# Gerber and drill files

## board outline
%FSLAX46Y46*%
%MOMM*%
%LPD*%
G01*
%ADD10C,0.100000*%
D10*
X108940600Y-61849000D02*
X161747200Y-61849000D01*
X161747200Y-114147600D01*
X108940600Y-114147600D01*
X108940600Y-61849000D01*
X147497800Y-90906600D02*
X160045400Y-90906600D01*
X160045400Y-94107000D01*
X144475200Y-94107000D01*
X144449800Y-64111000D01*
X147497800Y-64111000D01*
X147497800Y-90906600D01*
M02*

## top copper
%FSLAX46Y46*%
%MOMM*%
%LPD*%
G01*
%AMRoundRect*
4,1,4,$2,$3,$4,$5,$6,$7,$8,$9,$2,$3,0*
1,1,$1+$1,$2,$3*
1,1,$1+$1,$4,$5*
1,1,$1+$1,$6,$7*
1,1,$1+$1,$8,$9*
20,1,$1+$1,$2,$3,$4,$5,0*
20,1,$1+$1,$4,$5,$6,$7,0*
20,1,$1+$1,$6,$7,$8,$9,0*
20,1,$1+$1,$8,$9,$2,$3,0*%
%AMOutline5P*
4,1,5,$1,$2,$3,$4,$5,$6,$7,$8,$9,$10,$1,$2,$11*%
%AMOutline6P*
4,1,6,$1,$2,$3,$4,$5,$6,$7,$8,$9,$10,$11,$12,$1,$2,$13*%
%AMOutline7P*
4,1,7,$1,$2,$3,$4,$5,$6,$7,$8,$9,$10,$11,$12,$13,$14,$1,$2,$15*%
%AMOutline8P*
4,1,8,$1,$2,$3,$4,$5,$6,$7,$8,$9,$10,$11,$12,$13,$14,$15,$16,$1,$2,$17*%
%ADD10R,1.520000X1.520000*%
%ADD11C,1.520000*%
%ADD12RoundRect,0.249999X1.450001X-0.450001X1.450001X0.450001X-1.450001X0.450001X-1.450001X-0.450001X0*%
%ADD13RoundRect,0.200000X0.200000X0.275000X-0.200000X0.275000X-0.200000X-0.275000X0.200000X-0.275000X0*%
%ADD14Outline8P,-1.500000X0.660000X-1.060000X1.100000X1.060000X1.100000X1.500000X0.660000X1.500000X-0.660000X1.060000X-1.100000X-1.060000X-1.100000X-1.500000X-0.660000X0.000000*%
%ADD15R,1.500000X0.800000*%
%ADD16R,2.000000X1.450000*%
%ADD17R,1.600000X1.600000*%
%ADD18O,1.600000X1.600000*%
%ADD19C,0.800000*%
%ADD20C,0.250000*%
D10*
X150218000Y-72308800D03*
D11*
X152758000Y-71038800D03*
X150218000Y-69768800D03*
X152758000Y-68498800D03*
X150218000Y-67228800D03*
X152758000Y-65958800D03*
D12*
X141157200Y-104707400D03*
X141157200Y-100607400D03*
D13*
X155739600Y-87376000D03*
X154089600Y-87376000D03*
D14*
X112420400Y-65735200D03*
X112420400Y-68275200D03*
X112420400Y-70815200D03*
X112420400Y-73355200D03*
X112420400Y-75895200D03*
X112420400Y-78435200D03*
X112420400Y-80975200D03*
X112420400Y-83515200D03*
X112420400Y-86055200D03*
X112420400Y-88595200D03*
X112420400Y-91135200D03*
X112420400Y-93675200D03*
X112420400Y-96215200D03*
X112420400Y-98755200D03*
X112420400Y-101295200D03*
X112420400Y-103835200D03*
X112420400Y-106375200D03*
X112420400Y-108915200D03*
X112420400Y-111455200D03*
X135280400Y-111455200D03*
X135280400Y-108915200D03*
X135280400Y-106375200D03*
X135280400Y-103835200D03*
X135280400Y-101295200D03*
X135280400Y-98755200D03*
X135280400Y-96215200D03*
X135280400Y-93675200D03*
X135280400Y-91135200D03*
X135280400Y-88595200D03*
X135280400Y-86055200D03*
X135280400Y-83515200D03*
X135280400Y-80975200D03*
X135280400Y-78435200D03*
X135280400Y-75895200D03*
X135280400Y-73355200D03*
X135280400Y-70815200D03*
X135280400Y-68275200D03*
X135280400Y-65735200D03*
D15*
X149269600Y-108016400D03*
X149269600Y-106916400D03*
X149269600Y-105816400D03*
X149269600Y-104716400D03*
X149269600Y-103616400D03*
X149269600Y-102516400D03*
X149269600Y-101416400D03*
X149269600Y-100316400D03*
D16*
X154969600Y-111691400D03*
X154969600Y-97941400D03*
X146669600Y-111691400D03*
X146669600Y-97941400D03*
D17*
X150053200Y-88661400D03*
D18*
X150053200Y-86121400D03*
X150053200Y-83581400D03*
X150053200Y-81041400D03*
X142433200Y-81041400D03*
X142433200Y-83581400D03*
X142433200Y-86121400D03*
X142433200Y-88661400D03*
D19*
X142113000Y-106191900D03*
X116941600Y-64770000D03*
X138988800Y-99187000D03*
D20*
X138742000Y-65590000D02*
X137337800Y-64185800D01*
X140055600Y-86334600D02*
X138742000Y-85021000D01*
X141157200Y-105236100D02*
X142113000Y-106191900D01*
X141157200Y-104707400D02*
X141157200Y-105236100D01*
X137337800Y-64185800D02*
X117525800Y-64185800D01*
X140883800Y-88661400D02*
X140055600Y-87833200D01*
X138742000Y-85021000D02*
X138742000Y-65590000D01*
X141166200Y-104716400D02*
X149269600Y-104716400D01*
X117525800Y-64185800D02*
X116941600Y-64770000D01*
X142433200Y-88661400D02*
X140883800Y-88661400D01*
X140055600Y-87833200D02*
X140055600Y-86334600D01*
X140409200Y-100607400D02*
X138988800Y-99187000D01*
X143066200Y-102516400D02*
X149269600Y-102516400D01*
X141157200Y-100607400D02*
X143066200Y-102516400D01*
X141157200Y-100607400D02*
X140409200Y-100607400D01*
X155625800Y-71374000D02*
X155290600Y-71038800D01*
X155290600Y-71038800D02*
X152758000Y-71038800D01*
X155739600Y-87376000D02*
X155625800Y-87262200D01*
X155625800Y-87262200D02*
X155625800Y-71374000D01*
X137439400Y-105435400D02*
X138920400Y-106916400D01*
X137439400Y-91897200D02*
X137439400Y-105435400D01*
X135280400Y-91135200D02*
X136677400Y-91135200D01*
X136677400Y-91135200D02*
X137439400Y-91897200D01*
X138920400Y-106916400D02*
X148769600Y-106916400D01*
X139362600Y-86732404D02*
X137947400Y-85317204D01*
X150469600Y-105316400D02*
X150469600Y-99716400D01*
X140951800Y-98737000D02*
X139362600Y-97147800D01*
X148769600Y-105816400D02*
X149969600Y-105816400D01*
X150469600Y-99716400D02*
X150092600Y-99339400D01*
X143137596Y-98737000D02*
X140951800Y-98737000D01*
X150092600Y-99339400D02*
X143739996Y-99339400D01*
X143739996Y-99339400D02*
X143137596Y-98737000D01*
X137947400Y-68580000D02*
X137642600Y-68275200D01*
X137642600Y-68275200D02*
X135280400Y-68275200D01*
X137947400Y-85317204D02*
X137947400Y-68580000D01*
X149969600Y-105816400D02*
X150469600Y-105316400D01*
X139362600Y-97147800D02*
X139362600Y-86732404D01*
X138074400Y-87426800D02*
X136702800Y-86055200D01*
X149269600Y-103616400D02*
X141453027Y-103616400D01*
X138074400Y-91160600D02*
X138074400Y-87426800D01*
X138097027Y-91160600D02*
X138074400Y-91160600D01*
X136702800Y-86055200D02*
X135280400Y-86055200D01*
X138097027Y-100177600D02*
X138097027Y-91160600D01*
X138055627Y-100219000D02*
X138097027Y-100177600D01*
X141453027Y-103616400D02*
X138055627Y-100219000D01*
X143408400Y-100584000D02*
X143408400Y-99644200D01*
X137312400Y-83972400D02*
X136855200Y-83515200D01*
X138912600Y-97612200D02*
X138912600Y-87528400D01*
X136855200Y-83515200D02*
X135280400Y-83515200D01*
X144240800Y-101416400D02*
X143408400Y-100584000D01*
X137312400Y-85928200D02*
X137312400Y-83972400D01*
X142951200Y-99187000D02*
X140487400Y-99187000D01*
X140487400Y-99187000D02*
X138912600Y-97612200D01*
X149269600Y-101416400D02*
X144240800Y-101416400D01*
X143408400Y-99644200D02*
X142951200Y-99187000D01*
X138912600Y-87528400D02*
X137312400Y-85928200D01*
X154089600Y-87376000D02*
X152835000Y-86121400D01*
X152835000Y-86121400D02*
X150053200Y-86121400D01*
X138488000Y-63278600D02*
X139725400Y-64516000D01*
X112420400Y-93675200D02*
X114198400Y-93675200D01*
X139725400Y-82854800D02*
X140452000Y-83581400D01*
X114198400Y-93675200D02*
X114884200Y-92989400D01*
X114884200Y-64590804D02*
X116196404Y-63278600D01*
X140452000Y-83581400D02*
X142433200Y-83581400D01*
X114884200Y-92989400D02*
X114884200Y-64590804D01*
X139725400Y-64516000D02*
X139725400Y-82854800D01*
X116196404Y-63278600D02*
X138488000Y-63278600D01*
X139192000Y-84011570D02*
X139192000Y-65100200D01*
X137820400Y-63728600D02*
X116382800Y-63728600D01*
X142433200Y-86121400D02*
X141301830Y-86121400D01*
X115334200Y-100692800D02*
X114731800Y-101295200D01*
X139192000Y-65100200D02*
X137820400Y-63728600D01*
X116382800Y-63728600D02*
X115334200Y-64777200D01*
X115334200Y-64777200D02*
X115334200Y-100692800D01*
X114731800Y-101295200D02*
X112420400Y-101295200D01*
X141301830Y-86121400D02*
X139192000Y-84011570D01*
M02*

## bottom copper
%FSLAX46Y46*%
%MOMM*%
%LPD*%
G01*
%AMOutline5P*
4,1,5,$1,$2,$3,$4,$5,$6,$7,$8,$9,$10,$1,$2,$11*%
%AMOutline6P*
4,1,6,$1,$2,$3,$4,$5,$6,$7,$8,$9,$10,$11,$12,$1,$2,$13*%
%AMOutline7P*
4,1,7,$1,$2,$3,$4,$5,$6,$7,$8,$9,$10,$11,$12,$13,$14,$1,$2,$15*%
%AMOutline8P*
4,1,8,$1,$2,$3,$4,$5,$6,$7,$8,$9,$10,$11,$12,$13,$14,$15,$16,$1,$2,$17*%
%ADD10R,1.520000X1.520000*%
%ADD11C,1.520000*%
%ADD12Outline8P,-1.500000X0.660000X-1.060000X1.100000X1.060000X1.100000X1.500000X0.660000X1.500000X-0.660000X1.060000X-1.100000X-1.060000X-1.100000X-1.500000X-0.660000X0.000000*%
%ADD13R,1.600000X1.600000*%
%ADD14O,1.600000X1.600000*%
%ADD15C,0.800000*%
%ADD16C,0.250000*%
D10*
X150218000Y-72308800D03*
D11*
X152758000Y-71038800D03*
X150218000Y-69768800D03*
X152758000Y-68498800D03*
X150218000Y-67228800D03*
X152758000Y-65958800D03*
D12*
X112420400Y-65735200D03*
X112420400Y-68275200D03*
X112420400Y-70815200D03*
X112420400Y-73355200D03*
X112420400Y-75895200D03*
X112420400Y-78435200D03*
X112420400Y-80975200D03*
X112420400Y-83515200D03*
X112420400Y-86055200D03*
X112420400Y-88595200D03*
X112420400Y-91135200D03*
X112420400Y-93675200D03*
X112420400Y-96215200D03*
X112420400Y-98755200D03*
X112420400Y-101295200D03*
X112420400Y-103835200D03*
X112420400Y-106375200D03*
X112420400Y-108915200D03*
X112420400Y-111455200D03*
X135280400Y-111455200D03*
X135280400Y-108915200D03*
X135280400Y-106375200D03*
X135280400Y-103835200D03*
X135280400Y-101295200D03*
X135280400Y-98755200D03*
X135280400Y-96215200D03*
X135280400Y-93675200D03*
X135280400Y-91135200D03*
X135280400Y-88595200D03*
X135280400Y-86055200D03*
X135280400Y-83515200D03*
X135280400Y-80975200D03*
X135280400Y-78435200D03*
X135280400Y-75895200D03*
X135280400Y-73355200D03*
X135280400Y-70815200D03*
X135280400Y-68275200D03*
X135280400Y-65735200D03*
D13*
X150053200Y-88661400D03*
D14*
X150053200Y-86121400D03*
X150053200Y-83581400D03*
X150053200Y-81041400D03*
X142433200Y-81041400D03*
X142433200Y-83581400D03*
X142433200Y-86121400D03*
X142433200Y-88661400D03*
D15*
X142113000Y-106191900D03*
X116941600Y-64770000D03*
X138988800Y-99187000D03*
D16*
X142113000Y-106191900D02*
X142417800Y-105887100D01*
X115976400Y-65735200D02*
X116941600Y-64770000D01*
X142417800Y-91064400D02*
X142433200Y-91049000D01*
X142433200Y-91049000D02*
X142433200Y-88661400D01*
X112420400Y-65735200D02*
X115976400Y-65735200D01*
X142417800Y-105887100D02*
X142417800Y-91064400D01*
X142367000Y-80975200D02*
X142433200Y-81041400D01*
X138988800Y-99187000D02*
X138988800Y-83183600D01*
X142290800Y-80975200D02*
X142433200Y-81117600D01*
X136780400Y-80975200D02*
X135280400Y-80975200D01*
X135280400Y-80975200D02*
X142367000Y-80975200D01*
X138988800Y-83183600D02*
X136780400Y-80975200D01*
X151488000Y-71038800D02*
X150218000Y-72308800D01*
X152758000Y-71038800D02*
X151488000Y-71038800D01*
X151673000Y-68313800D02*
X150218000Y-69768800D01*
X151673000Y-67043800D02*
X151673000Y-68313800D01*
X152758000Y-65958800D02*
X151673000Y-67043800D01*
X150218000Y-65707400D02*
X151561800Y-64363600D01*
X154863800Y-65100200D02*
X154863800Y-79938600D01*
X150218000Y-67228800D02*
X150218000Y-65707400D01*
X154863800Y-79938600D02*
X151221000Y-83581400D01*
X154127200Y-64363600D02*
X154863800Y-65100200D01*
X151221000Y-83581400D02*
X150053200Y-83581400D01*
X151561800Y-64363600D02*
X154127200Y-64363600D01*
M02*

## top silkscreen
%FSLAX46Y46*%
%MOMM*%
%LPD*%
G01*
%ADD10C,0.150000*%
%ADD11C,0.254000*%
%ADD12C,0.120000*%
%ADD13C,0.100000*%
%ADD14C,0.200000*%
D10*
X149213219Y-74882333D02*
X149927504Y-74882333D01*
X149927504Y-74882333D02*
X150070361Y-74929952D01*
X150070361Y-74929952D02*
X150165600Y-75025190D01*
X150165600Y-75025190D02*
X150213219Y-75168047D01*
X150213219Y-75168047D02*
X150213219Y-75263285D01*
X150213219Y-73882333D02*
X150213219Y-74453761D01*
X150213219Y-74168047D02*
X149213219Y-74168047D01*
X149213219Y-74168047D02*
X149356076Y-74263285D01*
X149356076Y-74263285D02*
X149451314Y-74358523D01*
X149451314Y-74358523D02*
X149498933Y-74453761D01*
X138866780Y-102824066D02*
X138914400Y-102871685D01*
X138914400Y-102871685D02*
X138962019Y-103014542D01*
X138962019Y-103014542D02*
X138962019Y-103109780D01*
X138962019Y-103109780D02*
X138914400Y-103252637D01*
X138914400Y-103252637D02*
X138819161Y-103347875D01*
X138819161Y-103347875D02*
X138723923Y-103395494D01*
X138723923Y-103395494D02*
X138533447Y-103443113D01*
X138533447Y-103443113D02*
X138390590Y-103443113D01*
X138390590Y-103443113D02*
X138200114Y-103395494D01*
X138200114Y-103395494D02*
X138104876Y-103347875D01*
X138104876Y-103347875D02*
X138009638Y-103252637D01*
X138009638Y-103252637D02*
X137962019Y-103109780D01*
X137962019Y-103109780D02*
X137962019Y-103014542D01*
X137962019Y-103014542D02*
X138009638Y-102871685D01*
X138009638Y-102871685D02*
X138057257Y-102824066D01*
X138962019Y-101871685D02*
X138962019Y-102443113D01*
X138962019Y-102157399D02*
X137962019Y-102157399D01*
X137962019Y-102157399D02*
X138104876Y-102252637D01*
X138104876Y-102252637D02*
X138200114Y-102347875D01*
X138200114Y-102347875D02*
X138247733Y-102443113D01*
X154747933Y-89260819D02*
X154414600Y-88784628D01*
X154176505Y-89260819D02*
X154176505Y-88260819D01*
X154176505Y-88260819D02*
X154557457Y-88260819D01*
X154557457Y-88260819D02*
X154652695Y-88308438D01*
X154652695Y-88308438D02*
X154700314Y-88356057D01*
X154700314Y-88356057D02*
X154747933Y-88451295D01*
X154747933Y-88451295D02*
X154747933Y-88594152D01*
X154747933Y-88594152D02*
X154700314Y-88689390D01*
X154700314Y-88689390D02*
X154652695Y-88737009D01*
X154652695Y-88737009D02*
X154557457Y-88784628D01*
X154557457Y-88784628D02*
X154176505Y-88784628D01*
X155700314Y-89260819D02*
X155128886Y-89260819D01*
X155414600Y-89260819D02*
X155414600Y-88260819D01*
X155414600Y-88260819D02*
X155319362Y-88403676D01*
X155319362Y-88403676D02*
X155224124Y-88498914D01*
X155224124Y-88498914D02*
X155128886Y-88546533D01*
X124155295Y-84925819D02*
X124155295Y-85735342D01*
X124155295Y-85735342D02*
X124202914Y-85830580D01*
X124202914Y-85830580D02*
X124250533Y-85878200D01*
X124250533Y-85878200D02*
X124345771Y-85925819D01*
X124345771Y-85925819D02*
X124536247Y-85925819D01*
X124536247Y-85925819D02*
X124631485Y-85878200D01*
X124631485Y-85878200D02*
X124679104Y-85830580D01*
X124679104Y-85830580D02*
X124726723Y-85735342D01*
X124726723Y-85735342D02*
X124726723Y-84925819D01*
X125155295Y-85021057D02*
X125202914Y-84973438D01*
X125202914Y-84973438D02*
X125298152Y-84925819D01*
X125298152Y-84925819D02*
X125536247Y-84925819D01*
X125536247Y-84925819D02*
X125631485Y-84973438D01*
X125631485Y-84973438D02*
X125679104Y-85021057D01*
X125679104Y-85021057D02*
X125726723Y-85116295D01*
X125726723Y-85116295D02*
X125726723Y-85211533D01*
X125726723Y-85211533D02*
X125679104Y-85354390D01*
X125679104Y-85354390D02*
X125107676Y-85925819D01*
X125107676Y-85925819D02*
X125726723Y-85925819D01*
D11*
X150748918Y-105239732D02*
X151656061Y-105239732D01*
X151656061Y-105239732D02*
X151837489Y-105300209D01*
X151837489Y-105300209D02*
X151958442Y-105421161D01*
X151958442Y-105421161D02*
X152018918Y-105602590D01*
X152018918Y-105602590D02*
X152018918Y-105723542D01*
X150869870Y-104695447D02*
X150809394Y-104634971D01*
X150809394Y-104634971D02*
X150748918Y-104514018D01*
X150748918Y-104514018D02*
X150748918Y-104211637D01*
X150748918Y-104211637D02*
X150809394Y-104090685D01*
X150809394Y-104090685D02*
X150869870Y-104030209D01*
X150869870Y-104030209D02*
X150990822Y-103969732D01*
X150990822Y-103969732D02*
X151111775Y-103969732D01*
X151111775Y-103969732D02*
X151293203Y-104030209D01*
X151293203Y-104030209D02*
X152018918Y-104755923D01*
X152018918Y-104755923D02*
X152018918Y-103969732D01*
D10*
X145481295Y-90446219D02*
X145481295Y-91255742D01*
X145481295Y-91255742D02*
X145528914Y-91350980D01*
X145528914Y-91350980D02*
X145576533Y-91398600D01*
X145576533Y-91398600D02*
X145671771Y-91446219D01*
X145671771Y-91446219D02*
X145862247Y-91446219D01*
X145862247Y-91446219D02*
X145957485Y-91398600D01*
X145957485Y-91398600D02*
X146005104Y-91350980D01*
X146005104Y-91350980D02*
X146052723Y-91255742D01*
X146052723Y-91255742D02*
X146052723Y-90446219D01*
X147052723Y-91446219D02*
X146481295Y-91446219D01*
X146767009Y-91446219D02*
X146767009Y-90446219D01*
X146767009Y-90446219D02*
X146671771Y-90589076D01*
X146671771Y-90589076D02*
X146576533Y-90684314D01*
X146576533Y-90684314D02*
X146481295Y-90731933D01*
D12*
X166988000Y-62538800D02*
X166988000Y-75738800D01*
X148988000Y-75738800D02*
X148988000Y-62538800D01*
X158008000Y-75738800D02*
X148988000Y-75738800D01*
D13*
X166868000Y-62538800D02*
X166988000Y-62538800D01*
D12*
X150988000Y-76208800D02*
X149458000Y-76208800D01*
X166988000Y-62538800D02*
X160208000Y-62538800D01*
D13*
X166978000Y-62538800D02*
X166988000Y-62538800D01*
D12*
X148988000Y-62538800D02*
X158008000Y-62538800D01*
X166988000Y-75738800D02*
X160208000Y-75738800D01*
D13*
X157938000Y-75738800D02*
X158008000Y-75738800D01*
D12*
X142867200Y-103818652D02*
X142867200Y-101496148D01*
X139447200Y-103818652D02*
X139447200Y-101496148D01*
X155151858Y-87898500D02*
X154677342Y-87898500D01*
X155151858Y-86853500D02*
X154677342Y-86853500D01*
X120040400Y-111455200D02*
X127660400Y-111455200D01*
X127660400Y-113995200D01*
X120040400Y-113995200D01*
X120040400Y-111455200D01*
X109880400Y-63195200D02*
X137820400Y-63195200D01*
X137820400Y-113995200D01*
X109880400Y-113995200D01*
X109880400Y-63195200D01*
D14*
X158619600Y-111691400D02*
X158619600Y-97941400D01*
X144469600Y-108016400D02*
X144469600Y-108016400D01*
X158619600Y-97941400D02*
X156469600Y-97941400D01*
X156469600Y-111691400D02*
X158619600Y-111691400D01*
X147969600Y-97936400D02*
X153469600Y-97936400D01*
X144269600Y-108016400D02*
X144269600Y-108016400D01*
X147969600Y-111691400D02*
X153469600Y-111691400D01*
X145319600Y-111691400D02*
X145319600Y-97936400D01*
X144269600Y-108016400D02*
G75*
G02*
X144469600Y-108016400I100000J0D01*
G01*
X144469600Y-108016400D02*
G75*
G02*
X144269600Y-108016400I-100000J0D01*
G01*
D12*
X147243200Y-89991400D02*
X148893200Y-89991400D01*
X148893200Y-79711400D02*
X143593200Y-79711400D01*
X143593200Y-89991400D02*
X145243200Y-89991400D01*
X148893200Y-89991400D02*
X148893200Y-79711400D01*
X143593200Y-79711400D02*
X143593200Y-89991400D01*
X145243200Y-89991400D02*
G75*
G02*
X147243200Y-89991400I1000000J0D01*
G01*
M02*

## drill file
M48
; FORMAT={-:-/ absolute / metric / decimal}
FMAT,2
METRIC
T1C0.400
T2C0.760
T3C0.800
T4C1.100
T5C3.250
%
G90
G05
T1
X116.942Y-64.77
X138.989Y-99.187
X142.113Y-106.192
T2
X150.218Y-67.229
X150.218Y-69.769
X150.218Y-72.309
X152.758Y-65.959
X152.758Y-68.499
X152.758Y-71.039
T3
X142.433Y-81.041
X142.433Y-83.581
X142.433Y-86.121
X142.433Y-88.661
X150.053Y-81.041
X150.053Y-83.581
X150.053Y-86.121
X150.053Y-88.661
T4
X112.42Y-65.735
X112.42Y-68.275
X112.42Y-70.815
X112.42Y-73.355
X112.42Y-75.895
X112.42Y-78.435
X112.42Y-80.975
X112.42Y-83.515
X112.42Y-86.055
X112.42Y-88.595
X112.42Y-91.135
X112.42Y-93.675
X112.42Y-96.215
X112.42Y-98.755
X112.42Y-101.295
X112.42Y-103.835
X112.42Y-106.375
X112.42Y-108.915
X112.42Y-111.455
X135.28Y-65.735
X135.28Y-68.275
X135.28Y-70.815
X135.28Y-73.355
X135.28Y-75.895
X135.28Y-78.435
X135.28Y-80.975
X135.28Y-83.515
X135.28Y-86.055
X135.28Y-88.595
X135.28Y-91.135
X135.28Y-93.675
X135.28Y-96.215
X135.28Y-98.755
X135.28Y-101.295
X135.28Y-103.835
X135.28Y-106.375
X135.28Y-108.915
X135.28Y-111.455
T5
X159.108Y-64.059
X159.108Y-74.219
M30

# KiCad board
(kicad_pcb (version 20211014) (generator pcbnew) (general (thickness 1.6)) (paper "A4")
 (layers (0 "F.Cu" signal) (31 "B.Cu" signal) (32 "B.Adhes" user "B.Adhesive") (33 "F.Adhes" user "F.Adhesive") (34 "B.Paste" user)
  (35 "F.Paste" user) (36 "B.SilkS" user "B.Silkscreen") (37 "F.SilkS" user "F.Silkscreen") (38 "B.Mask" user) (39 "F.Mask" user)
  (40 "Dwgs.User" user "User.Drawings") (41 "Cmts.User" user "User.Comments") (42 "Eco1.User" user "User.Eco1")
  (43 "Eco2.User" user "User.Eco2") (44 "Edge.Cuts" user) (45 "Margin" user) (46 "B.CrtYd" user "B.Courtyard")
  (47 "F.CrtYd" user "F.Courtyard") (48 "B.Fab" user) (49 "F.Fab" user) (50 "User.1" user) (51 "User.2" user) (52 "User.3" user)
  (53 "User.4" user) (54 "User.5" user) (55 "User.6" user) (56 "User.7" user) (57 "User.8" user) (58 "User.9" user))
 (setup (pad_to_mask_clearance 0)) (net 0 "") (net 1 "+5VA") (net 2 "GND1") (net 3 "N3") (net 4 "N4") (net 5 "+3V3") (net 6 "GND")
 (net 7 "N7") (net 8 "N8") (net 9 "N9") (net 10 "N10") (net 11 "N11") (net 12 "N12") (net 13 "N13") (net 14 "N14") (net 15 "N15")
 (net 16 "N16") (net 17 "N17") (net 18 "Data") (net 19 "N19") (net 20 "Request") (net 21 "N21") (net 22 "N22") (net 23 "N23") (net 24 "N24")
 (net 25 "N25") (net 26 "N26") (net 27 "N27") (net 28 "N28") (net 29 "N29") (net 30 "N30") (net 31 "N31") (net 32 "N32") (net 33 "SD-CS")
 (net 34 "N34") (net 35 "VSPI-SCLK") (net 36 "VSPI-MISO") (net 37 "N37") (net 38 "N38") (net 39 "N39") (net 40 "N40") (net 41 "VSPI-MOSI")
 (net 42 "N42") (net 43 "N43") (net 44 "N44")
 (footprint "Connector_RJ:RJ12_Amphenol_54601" (layer "F.Cu") (at 150.218 72.3088 90)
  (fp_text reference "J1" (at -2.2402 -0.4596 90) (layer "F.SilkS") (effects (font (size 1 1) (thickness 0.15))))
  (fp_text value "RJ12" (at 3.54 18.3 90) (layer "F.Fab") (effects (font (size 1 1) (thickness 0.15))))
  (fp_line (start 9.77 16.77) (end -3.43 16.77) (layer "F.SilkS") (width 0.12))
  (fp_line (start -3.43 -1.23) (end 9.77 -1.23) (layer "F.SilkS") (width 0.12))
  (fp_line (start -3.43 7.79) (end -3.43 -1.23) (layer "F.SilkS") (width 0.12))
  (fp_line (start 9.77 16.65) (end 9.77 16.77) (layer "F.SilkS") (width 0.1))
  (fp_line (start -3.9 0.77) (end -3.9 -0.76) (layer "F.SilkS") (width 0.12))
  (fp_line (start 9.77 16.77) (end 9.77 9.99) (layer "F.SilkS") (width 0.12))
  (fp_line (start 9.77 16.76) (end 9.77 16.77) (layer "F.SilkS") (width 0.1))
  (fp_line (start 9.77 -1.23) (end 9.77 7.79) (layer "F.SilkS") (width 0.12))
  (fp_line (start -3.43 16.77) (end -3.43 9.99) (layer "F.SilkS") (width 0.12))
  (fp_line (start -3.43 7.72) (end -3.43 7.79) (layer "F.SilkS") (width 0.1))
  (pad "" np_thru_hole circle (at -1.91 8.89 90) (size 3.25 3.25) (drill 3.25) (layers *.Cu *.Mask))
  (pad "" np_thru_hole circle (at 8.25 8.89 90) (size 3.25 3.25) (drill 3.25) (layers *.Cu *.Mask))
  (pad "1" thru_hole rect (at 0 0 90) (size 1.52 1.52) (drill 0.76) (layers *.Cu *.Mask) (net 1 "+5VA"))
  (pad "2" thru_hole circle (at 1.27 2.54 90) (size 1.52 1.52) (drill 0.76) (layers *.Cu *.Mask) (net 1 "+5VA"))
  (pad "3" thru_hole circle (at 2.54 0 90) (size 1.52 1.52) (drill 0.76) (layers *.Cu *.Mask) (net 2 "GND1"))
  (pad "4" thru_hole circle (at 3.81 2.54 90) (size 1.52 1.52) (drill 0.76) (layers *.Cu *.Mask) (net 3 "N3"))
  (pad "5" thru_hole circle (at 5.08 0 90) (size 1.52 1.52) (drill 0.76) (layers *.Cu *.Mask) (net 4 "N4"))
  (pad "6" thru_hole circle (at 6.35 2.54 90) (size 1.52 1.52) (drill 0.76) (layers *.Cu *.Mask) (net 2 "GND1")))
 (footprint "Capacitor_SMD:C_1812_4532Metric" (layer "F.Cu") (at 141.1572 102.6574 90)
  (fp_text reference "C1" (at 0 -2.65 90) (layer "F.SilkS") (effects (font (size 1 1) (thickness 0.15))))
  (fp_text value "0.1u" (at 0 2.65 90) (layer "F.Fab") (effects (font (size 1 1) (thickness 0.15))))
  (fp_line (start -1.161252 1.71) (end 1.161252 1.71) (layer "F.SilkS") (width 0.12))
  (fp_line (start -1.161252 -1.71) (end 1.161252 -1.71) (layer "F.SilkS") (width 0.12))
  (pad "1" smd roundrect (at -2.05 0 90) (size 1.4 3.4) (layers "F.Cu" "F.Paste" "F.Mask") (roundrect_rratio 0.178571) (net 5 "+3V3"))
  (pad "2" smd roundrect (at 2.05 0 90) (size 1.4 3.4) (layers "F.Cu" "F.Paste" "F.Mask") (roundrect_rratio 0.178571) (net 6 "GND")))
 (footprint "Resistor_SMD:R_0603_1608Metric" (layer "F.Cu") (at 154.9146 87.376 180)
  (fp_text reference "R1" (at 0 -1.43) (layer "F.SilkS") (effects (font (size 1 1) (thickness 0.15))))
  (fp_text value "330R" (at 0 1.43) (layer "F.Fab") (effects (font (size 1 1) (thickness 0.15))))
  (fp_line (start -0.237258 -0.5225) (end 0.237258 -0.5225) (layer "F.SilkS") (width 0.12))
  (fp_line (start -0.237258 0.5225) (end 0.237258 0.5225) (layer "F.SilkS") (width 0.12))
  (pad "1" smd roundrect (at -0.825 0 180) (size 0.8 0.95) (layers "F.Cu" "F.Paste" "F.Mask") (roundrect_rratio 0.25) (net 1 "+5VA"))
  (pad "2" smd roundrect (at 0.825 0 180) (size 0.8 0.95) (layers "F.Cu" "F.Paste" "F.Mask") (roundrect_rratio 0.25) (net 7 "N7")))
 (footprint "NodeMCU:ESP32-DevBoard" (layer "F.Cu") (at 112.4204 80.9752)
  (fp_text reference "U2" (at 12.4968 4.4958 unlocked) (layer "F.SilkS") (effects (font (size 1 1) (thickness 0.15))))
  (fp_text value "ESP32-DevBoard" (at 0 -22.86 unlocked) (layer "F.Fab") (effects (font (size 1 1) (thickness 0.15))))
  (fp_rect (start 7.62 30.48) (end 15.24 33.02) (layer "F.SilkS") (width 0.12) (fill none))
  (fp_rect (start -2.54 -17.78) (end 25.4 33.02) (layer "F.SilkS") (width 0.12) (fill none))
  (pad "1" thru_hole roundrect (at 0 -15.24) (size 3 2.2) (drill 1.1) (layers *.Cu *.Mask) (roundrect_rratio 0) (chamfer_ratio 0.2)
   (chamfer top_left top_right bottom_left bottom_right) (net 5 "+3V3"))
  (pad "2" thru_hole roundrect (at 0 -12.7) (size 3 2.2) (drill 1.1) (layers *.Cu *.Mask) (roundrect_rratio 0) (chamfer_ratio 0.2)
   (chamfer top_left top_right bottom_left bottom_right) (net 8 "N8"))
  (pad "3" thru_hole roundrect (at 0 -10.16) (size 3 2.2) (drill 1.1) (layers *.Cu *.Mask) (roundrect_rratio 0) (chamfer_ratio 0.2)
   (chamfer top_left top_right bottom_left bottom_right) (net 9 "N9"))
  (pad "4" thru_hole roundrect (at 0 -7.62) (size 3 2.2) (drill 1.1) (layers *.Cu *.Mask) (roundrect_rratio 0) (chamfer_ratio 0.2)
   (chamfer top_left top_right bottom_left bottom_right) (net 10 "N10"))
  (pad "5" thru_hole roundrect (at 0 -5.08) (size 3 2.2) (drill 1.1) (layers *.Cu *.Mask) (roundrect_rratio 0) (chamfer_ratio 0.2)
   (chamfer top_left top_right bottom_left bottom_right) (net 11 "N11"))
  (pad "6" thru_hole roundrect (at 0 -2.54) (size 3 2.2) (drill 1.1) (layers *.Cu *.Mask) (roundrect_rratio 0) (chamfer_ratio 0.2)
   (chamfer top_left top_right bottom_left bottom_right) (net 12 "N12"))
  (pad "7" thru_hole roundrect (at 0 0) (size 3 2.2) (drill 1.1) (layers *.Cu *.Mask) (roundrect_rratio 0) (chamfer_ratio 0.2)
   (chamfer top_left top_right bottom_left bottom_right) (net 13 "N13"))
  (pad "8" thru_hole roundrect (at 0 2.54) (size 3 2.2) (drill 1.1) (layers *.Cu *.Mask) (roundrect_rratio 0) (chamfer_ratio 0.2)
   (chamfer top_left top_right bottom_left bottom_right) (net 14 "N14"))
  (pad "9" thru_hole roundrect (at 0 5.08) (size 3 2.2) (drill 1.1) (layers *.Cu *.Mask) (roundrect_rratio 0) (chamfer_ratio 0.2)
   (chamfer top_left top_right bottom_left bottom_right) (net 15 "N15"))
  (pad "10" thru_hole roundrect (at 0 7.62) (size 3 2.2) (drill 1.1) (layers *.Cu *.Mask) (roundrect_rratio 0) (chamfer_ratio 0.2)
   (chamfer top_left top_right bottom_left bottom_right) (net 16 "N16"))
  (pad "11" thru_hole roundrect (at 0 10.16) (size 3 2.2) (drill 1.1) (layers *.Cu *.Mask) (roundrect_rratio 0) (chamfer_ratio 0.2)
   (chamfer top_left top_right bottom_left bottom_right) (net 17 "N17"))
  (pad "12" thru_hole roundrect (at 0 12.7) (size 3 2.2) (drill 1.1) (layers *.Cu *.Mask) (roundrect_rratio 0) (chamfer_ratio 0.2)
   (chamfer top_left top_right bottom_left bottom_right) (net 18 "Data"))
  (pad "13" thru_hole roundrect (at 0 15.24) (size 3 2.2) (drill 1.1) (layers *.Cu *.Mask) (roundrect_rratio 0) (chamfer_ratio 0.2)
   (chamfer top_left top_right bottom_left bottom_right) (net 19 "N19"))
  (pad "14" thru_hole roundrect (at 0 17.78) (size 3 2.2) (drill 1.1) (layers *.Cu *.Mask) (roundrect_rratio 0) (chamfer_ratio 0.2)
   (chamfer top_left top_right bottom_left bottom_right) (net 6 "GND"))
  (pad "15" thru_hole roundrect (at 0 20.32) (size 3 2.2) (drill 1.1) (layers *.Cu *.Mask) (roundrect_rratio 0) (chamfer_ratio 0.2)
   (chamfer top_left top_right bottom_left bottom_right) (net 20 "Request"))
  (pad "16" thru_hole roundrect (at 0 22.86) (size 3 2.2) (drill 1.1) (layers *.Cu *.Mask) (roundrect_rratio 0) (chamfer_ratio 0.2)
   (chamfer top_left top_right bottom_left bottom_right) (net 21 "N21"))
  (pad "17" thru_hole roundrect (at 0 25.4) (size 3 2.2) (drill 1.1) (layers *.Cu *.Mask) (roundrect_rratio 0) (chamfer_ratio 0.2)
   (chamfer top_left top_right bottom_left bottom_right) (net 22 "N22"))
  (pad "18" thru_hole roundrect (at 0 27.94) (size 3 2.2) (drill 1.1) (layers *.Cu *.Mask) (roundrect_rratio 0) (chamfer_ratio 0.2)
   (chamfer top_left top_right bottom_left bottom_right) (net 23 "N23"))
  (pad "19" thru_hole roundrect (at 0 30.48) (size 3 2.2) (drill 1.1) (layers *.Cu *.Mask) (roundrect_rratio 0) (chamfer_ratio 0.2)
   (chamfer top_left top_right bottom_left bottom_right) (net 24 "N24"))
  (pad "20" thru_hole roundrect (at 22.86 30.48) (size 3 2.2) (drill 1.1) (layers *.Cu *.Mask) (roundrect_rratio 0) (chamfer_ratio 0.2)
   (chamfer top_left top_right bottom_left bottom_right) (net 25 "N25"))
  (pad "21" thru_hole roundrect (at 22.86 27.94) (size 3 2.2) (drill 1.1) (layers *.Cu *.Mask) (roundrect_rratio 0) (chamfer_ratio 0.2)
   (chamfer top_left top_right bottom_left bottom_right) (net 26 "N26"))
  (pad "22" thru_hole roundrect (at 22.86 25.4) (size 3 2.2) (drill 1.1) (layers *.Cu *.Mask) (roundrect_rratio 0) (chamfer_ratio 0.2)
   (chamfer top_left top_right bottom_left bottom_right) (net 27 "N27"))
  (pad "23" thru_hole roundrect (at 22.86 22.86) (size 3 2.2) (drill 1.1) (layers *.Cu *.Mask) (roundrect_rratio 0) (chamfer_ratio 0.2)
   (chamfer top_left top_right bottom_left bottom_right) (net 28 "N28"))
  (pad "24" thru_hole roundrect (at 22.86 20.32) (size 3 2.2) (drill 1.1) (layers *.Cu *.Mask) (roundrect_rratio 0) (chamfer_ratio 0.2)
   (chamfer top_left top_right bottom_left bottom_right) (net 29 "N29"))
  (pad "25" thru_hole roundrect (at 22.86 17.78) (size 3 2.2) (drill 1.1) (layers *.Cu *.Mask) (roundrect_rratio 0) (chamfer_ratio 0.2)
   (chamfer top_left top_right bottom_left bottom_right) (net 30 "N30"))
  (pad "26" thru_hole roundrect (at 22.86 15.24) (size 3 2.2) (drill 1.1) (layers *.Cu *.Mask) (roundrect_rratio 0) (chamfer_ratio 0.2)
   (chamfer top_left top_right bottom_left bottom_right) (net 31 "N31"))
  (pad "27" thru_hole roundrect (at 22.86 12.7) (size 3 2.2) (drill 1.1) (layers *.Cu *.Mask) (roundrect_rratio 0) (chamfer_ratio 0.2)
   (chamfer top_left top_right bottom_left bottom_right) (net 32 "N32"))
  (pad "28" thru_hole roundrect (at 22.86 10.16) (size 3 2.2) (drill 1.1) (layers *.Cu *.Mask) (roundrect_rratio 0) (chamfer_ratio 0.2)
   (chamfer top_left top_right bottom_left bottom_right) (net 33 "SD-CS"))
  (pad "29" thru_hole roundrect (at 22.86 7.62) (size 3 2.2) (drill 1.1) (layers *.Cu *.Mask) (roundrect_rratio 0) (chamfer_ratio 0.2)
   (chamfer top_left top_right bottom_left bottom_right) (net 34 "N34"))
  (pad "30" thru_hole roundrect (at 22.86 5.08) (size 3 2.2) (drill 1.1) (layers *.Cu *.Mask) (roundrect_rratio 0) (chamfer_ratio 0.2)
   (chamfer top_left top_right bottom_left bottom_right) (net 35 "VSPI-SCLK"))
  (pad "31" thru_hole roundrect (at 22.86 2.54) (size 3 2.2) (drill 1.1) (layers *.Cu *.Mask) (roundrect_rratio 0) (chamfer_ratio 0.2)
   (chamfer top_left top_right bottom_left bottom_right) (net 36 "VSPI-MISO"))
  (pad "32" thru_hole roundrect (at 22.86 0) (size 3 2.2) (drill 1.1) (layers *.Cu *.Mask) (roundrect_rratio 0) (chamfer_ratio 0.2)
   (chamfer top_left top_right bottom_left bottom_right) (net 6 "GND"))
  (pad "33" thru_hole roundrect (at 22.86 -2.54) (size 3 2.2) (drill 1.1) (layers *.Cu *.Mask) (roundrect_rratio 0) (chamfer_ratio 0.2)
   (chamfer top_left top_right bottom_left bottom_right) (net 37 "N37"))
  (pad "34" thru_hole roundrect (at 22.86 -5.08) (size 3 2.2) (drill 1.1) (layers *.Cu *.Mask) (roundrect_rratio 0) (chamfer_ratio 0.2)
   (chamfer top_left top_right bottom_left bottom_right) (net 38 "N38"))
  (pad "35" thru_hole roundrect (at 22.86 -7.62) (size 3 2.2) (drill 1.1) (layers *.Cu *.Mask) (roundrect_rratio 0) (chamfer_ratio 0.2)
   (chamfer top_left top_right bottom_left bottom_right) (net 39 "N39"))
  (pad "36" thru_hole roundrect (at 22.86 -10.16) (size 3 2.2) (drill 1.1) (layers *.Cu *.Mask) (roundrect_rratio 0) (chamfer_ratio 0.2)
   (chamfer top_left top_right bottom_left bottom_right) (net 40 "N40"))
  (pad "37" thru_hole roundrect (at 22.86 -12.7) (size 3 2.2) (drill 1.1) (layers *.Cu *.Mask) (roundrect_rratio 0) (chamfer_ratio 0.2)
   (chamfer top_left top_right bottom_left bottom_right) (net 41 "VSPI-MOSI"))
  (pad "38" thru_hole roundrect (at 22.86 -15.24) (size 3 2.2) (drill 1.1) (layers *.Cu *.Mask) (roundrect_rratio 0) (chamfer_ratio 0.2)
   (chamfer top_left top_right bottom_left bottom_right) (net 6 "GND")))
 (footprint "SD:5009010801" (layer "F.Cu") (at 151.9696 104.8164 90)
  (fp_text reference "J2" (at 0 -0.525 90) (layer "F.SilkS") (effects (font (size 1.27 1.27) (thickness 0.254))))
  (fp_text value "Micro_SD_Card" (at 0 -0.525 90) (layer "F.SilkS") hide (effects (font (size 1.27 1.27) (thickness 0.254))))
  (fp_line (start -6.875 6.65) (end 6.875 6.65) (layer "F.SilkS") (width 0.2))
  (fp_line (start -3.2 -7.5) (end -3.2 -7.5) (layer "F.SilkS") (width 0.2))
  (fp_line (start 6.875 6.65) (end 6.875 4.5) (layer "F.SilkS") (width 0.2))
  (fp_line (start -6.875 4.5) (end -6.875 6.65) (layer "F.SilkS") (width 0.2))
  (fp_line (start 6.88 -4) (end 6.88 1.5) (layer "F.SilkS") (width 0.2))
  (fp_line (start -3.2 -7.7) (end -3.2 -7.7) (layer "F.SilkS") (width 0.2))
  (fp_line (start -6.875 -4) (end -6.875 1.5) (layer "F.SilkS") (width 0.2))
  (fp_line (start -6.875 -6.65) (end 6.88 -6.65) (layer "F.SilkS") (width 0.2))
  (fp_arc (start -3.2 -7.7) (mid -3.1 -7.6) (end -3.2 -7.5) (layer "F.SilkS") (width 0.2))
  (fp_arc (start -3.2 -7.5) (mid -3.3 -7.6) (end -3.2 -7.7) (layer "F.SilkS") (width 0.2))
  (pad "1" smd rect locked (at -3.2 -2.7 90) (size 0.8 1.5) (layers "F.Cu" "F.Paste" "F.Mask") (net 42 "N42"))
  (pad "2" smd rect locked (at -2.1 -2.7 90) (size 0.8 1.5) (layers "F.Cu" "F.Paste" "F.Mask") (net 33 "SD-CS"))
  (pad "3" smd rect locked (at -1 -2.7 90) (size 0.8 1.5) (layers "F.Cu" "F.Paste" "F.Mask") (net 41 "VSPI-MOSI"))
  (pad "4" smd rect locked (at 0.1 -2.7 90) (size 0.8 1.5) (layers "F.Cu" "F.Paste" "F.Mask") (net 5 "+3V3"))
  (pad "5" smd rect locked (at 1.2 -2.7 90) (size 0.8 1.5) (layers "F.Cu" "F.Paste" "F.Mask") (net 35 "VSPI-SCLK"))
  (pad "6" smd rect locked (at 2.3 -2.7 90) (size 0.8 1.5) (layers "F.Cu" "F.Paste" "F.Mask") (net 6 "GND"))
  (pad "7" smd rect locked (at 3.4 -2.7 90) (size 0.8 1.5) (layers "F.Cu" "F.Paste" "F.Mask") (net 36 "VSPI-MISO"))
  (pad "8" smd rect locked (at 4.5 -2.7 90) (size 0.8 1.5) (layers "F.Cu" "F.Paste" "F.Mask") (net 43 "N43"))
  (pad "MP1" smd rect locked (at -6.875 3 90) (size 1.45 2) (layers "F.Cu" "F.Paste" "F.Mask"))
  (pad "MP2" smd rect locked (at 6.875 3 90) (size 1.45 2) (layers "F.Cu" "F.Paste" "F.Mask"))
  (pad "MP3" smd rect locked (at -6.875 -5.3 90) (size 1.45 2) (layers "F.Cu" "F.Paste" "F.Mask"))
  (pad "MP4" smd rect locked (at 6.875 -5.3 90) (size 1.45 2) (layers "F.Cu" "F.Paste" "F.Mask")))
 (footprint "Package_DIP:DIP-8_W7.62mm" (layer "F.Cu") (at 150.0532 88.6614 180)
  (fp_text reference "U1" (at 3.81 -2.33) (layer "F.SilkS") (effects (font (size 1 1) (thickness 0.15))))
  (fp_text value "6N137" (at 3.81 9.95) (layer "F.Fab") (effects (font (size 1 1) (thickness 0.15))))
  (fp_line (start 2.81 -1.33) (end 1.16 -1.33) (layer "F.SilkS") (width 0.12))
  (fp_line (start 1.16 8.95) (end 6.46 8.95) (layer "F.SilkS") (width 0.12))
  (fp_line (start 6.46 -1.33) (end 4.81 -1.33) (layer "F.SilkS") (width 0.12))
  (fp_line (start 1.16 -1.33) (end 1.16 8.95) (layer "F.SilkS") (width 0.12))
  (fp_line (start 6.46 8.95) (end 6.46 -1.33) (layer "F.SilkS") (width 0.12))
  (fp_arc (start 4.81 -1.33) (mid 3.81 -0.33) (end 2.81 -1.33) (layer "F.SilkS") (width 0.12))
  (pad "1" thru_hole rect (at 0 0 180) (size 1.6 1.6) (drill 0.8) (layers *.Cu *.Mask) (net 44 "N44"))
  (pad "2" thru_hole oval (at 0 2.54 180) (size 1.6 1.6) (drill 0.8) (layers *.Cu *.Mask) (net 7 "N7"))
  (pad "3" thru_hole oval (at 0 5.08 180) (size 1.6 1.6) (drill 0.8) (layers *.Cu *.Mask) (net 4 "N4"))
  (pad "4" thru_hole oval (at 0 7.62 180) (size 1.6 1.6) (drill 0.8) (layers *.Cu *.Mask))
  (pad "5" thru_hole oval (at 7.62 7.62 180) (size 1.6 1.6) (drill 0.8) (layers *.Cu *.Mask) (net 6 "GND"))
  (pad "6" thru_hole oval (at 7.62 5.08 180) (size 1.6 1.6) (drill 0.8) (layers *.Cu *.Mask) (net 18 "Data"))
  (pad "7" thru_hole oval (at 7.62 2.54 180) (size 1.6 1.6) (drill 0.8) (layers *.Cu *.Mask) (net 20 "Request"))
  (pad "8" thru_hole oval (at 7.62 0 180) (size 1.6 1.6) (drill 0.8) (layers *.Cu *.Mask) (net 5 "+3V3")))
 (gr_rect (start 108.9406 61.849) (end 161.7472 114.1476) (layer "Edge.Cuts") (width 0.1) (fill none))
 (gr_poly
  (pts (xy 147.4978 90.9066) (xy 160.0454 90.9066) (xy 160.0454 94.107) (xy 144.4752 94.107) (xy 144.4498 64.111) (xy 147.4978 64.111))
  (layer "Edge.Cuts") (width 0.1) (fill none))
 (segment (start 138.742 65.59) (end 137.3378 64.1858) (width 0.25) (layer "F.Cu") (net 5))
 (segment (start 140.0556 86.3346) (end 138.742 85.021) (width 0.25) (layer "F.Cu") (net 5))
 (segment (start 141.1572 105.2361) (end 142.113 106.1919) (width 0.25) (layer "F.Cu") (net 5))
 (segment (start 141.1572 104.7074) (end 141.1572 105.2361) (width 0.25) (layer "F.Cu") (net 5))
 (segment (start 137.3378 64.1858) (end 117.5258 64.1858) (width 0.25) (layer "F.Cu") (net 5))
 (segment (start 140.8838 88.6614) (end 140.0556 87.8332) (width 0.25) (layer "F.Cu") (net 5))
 (segment (start 138.742 85.021) (end 138.742 65.59) (width 0.25) (layer "F.Cu") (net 5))
 (segment (start 141.1662 104.7164) (end 149.2696 104.7164) (width 0.25) (layer "F.Cu") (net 5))
 (segment (start 117.5258 64.1858) (end 116.9416 64.77) (width 0.25) (layer "F.Cu") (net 5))
 (segment (start 142.4332 88.6614) (end 140.8838 88.6614) (width 0.25) (layer "F.Cu") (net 5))
 (segment (start 140.0556 87.8332) (end 140.0556 86.3346) (width 0.25) (layer "F.Cu") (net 5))
 (via (at 142.113 106.1919) (size 0.8) (drill 0.4) (layers "F.Cu" "B.Cu") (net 5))
 (via (at 116.9416 64.77) (size 0.8) (drill 0.4) (layers "F.Cu" "B.Cu") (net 5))
 (segment (start 142.113 106.1919) (end 142.4178 105.8871) (width 0.25) (layer "B.Cu") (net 5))
 (segment (start 115.9764 65.7352) (end 116.9416 64.77) (width 0.25) (layer "B.Cu") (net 5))
 (segment (start 142.4178 91.0644) (end 142.4332 91.049) (width 0.25) (layer "B.Cu") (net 5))
 (segment (start 142.4332 91.049) (end 142.4332 88.6614) (width 0.25) (layer "B.Cu") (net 5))
 (segment (start 112.4204 65.7352) (end 115.9764 65.7352) (width 0.25) (layer "B.Cu") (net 5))
 (segment (start 142.4178 105.8871) (end 142.4178 91.0644) (width 0.25) (layer "B.Cu") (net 5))
 (segment (start 140.4092 100.6074) (end 138.9888 99.187) (width 0.25) (layer "F.Cu") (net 6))
 (segment (start 143.0662 102.5164) (end 149.2696 102.5164) (width 0.25) (layer "F.Cu") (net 6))
 (segment (start 141.1572 100.6074) (end 143.0662 102.5164) (width 0.25) (layer "F.Cu") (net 6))
 (segment (start 141.1572 100.6074) (end 140.4092 100.6074) (width 0.25) (layer "F.Cu") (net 6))
 (via (at 138.9888 99.187) (size 0.8) (drill 0.4) (layers "F.Cu" "B.Cu") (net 6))
 (segment (start 142.367 80.9752) (end 142.4332 81.0414) (width 0.25) (layer "B.Cu") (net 6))
 (segment (start 138.9888 99.187) (end 138.9888 83.1836) (width 0.25) (layer "B.Cu") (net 6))
 (segment (start 142.2908 80.9752) (end 142.4332 81.1176) (width 0.25) (layer "B.Cu") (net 6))
 (segment (start 136.7804 80.9752) (end 135.2804 80.9752) (width 0.25) (layer "B.Cu") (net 6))
 (segment (start 135.2804 80.9752) (end 142.367 80.9752) (width 0.25) (layer "B.Cu") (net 6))
 (segment (start 138.9888 83.1836) (end 136.7804 80.9752) (width 0.25) (layer "B.Cu") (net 6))
 (segment (start 155.6258 71.374) (end 155.2906 71.0388) (width 0.25) (layer "F.Cu") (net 1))
 (segment (start 155.2906 71.0388) (end 152.758 71.0388) (width 0.25) (layer "F.Cu") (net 1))
 (segment (start 155.7396 87.376) (end 155.6258 87.2622) (width 0.25) (layer "F.Cu") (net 1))
 (segment (start 155.6258 87.2622) (end 155.6258 71.374) (width 0.25) (layer "F.Cu") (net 1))
 (segment (start 151.488 71.0388) (end 150.218 72.3088) (width 0.25) (layer "B.Cu") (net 1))
 (segment (start 152.758 71.0388) (end 151.488 71.0388) (width 0.25) (layer "B.Cu") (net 1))
 (segment (start 151.673 68.3138) (end 150.218 69.7688) (width 0.25) (layer "B.Cu") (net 2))
 (segment (start 151.673 67.0438) (end 151.673 68.3138) (width 0.25) (layer "B.Cu") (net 2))
 (segment (start 152.758 65.9588) (end 151.673 67.0438) (width 0.25) (layer "B.Cu") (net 2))
 (segment (start 150.218 65.7074) (end 151.5618 64.3636) (width 0.25) (layer "B.Cu") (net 4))
 (segment (start 154.8638 65.1002) (end 154.8638 79.9386) (width 0.25) (layer "B.Cu") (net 4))
 (segment (start 150.218 67.2288) (end 150.218 65.7074) (width 0.25) (layer "B.Cu") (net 4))
 (segment (start 154.8638 79.9386) (end 151.221 83.5814) (width 0.25) (layer "B.Cu") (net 4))
 (segment (start 154.1272 64.3636) (end 154.8638 65.1002) (width 0.25) (layer "B.Cu") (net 4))
 (segment (start 151.221 83.5814) (end 150.0532 83.5814) (width 0.25) (layer "B.Cu") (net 4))
 (segment (start 151.5618 64.3636) (end 154.1272 64.3636) (width 0.25) (layer "B.Cu") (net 4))
 (segment (start 137.4394 105.4354) (end 138.9204 106.9164) (width 0.25) (layer "F.Cu") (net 33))
 (segment (start 137.4394 91.8972) (end 137.4394 105.4354) (width 0.25) (layer "F.Cu") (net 33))
 (segment (start 135.2804 91.1352) (end 136.6774 91.1352) (width 0.25) (layer "F.Cu") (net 33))
 (segment (start 136.6774 91.1352) (end 137.4394 91.8972) (width 0.25) (layer "F.Cu") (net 33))
 (segment (start 138.9204 106.9164) (end 148.7696 106.9164) (width 0.25) (layer "F.Cu") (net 33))
 (segment (start 139.3626 86.732404) (end 137.9474 85.317204) (width 0.25) (layer "F.Cu") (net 41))
 (segment (start 150.4696 105.3164) (end 150.4696 99.7164) (width 0.25) (layer "F.Cu") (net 41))
 (segment (start 140.9518 98.737) (end 139.3626 97.1478) (width 0.25) (layer "F.Cu") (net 41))
 (segment (start 148.7696 105.8164) (end 149.9696 105.8164) (width 0.25) (layer "F.Cu") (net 41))
 (segment (start 150.4696 99.7164) (end 150.0926 99.3394) (width 0.25) (layer "F.Cu") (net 41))
 (segment (start 143.137596 98.737) (end 140.9518 98.737) (width 0.25) (layer "F.Cu") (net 41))
 (segment (start 150.0926 99.3394) (end 143.739996 99.3394) (width 0.25) (layer "F.Cu") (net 41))
 (segment (start 143.739996 99.3394) (end 143.137596 98.737) (width 0.25) (layer "F.Cu") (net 41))
 (segment (start 137.9474 68.58) (end 137.6426 68.2752) (width 0.25) (layer "F.Cu") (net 41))
 (segment (start 137.6426 68.2752) (end 135.2804 68.2752) (width 0.25) (layer "F.Cu") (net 41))
 (segment (start 137.9474 85.317204) (end 137.9474 68.58) (width 0.25) (layer "F.Cu") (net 41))
 (segment (start 149.9696 105.8164) (end 150.4696 105.3164) (width 0.25) (layer "F.Cu") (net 41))
 (segment (start 139.3626 97.1478) (end 139.3626 86.732404) (width 0.25) (layer "F.Cu") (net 41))
 (segment (start 138.0744 87.4268) (end 136.7028 86.0552) (width 0.25) (layer "F.Cu") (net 35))
 (segment (start 149.2696 103.6164) (end 141.453027 103.6164) (width 0.25) (layer "F.Cu") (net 35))
 (segment (start 138.0744 91.1606) (end 138.0744 87.4268) (width 0.25) (layer "F.Cu") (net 35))
 (segment (start 138.097027 91.1606) (end 138.0744 91.1606) (width 0.25) (layer "F.Cu") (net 35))
 (segment (start 136.7028 86.0552) (end 135.2804 86.0552) (width 0.25) (layer "F.Cu") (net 35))
 (segment (start 138.097027 100.1776) (end 138.097027 91.1606) (width 0.25) (layer "F.Cu") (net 35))
 (segment (start 138.055627 100.219) (end 138.097027 100.1776) (width 0.25) (layer "F.Cu") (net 35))
 (segment (start 141.453027 103.6164) (end 138.055627 100.219) (width 0.25) (layer "F.Cu") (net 35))
 (segment (start 143.4084 100.584) (end 143.4084 99.6442) (width 0.25) (layer "F.Cu") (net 36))
 (segment (start 137.3124 83.9724) (end 136.8552 83.5152) (width 0.25) (layer "F.Cu") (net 36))
 (segment (start 138.9126 97.6122) (end 138.9126 87.5284) (width 0.25) (layer "F.Cu") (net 36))
 (segment (start 136.8552 83.5152) (end 135.2804 83.5152) (width 0.25) (layer "F.Cu") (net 36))
 (segment (start 144.2408 101.4164) (end 143.4084 100.584) (width 0.25) (layer "F.Cu") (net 36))
 (segment (start 137.3124 85.9282) (end 137.3124 83.9724) (width 0.25) (layer "F.Cu") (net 36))
 (segment (start 142.9512 99.187) (end 140.4874 99.187) (width 0.25) (layer "F.Cu") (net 36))
 (segment (start 140.4874 99.187) (end 138.9126 97.6122) (width 0.25) (layer "F.Cu") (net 36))
 (segment (start 149.2696 101.4164) (end 144.2408 101.4164) (width 0.25) (layer "F.Cu") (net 36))
 (segment (start 143.4084 99.6442) (end 142.9512 99.187) (width 0.25) (layer "F.Cu") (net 36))
 (segment (start 138.9126 87.5284) (end 137.3124 85.9282) (width 0.25) (layer "F.Cu") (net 36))
 (segment (start 154.0896 87.376) (end 152.835 86.1214) (width 0.25) (layer "F.Cu") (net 7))
 (segment (start 152.835 86.1214) (end 150.0532 86.1214) (width 0.25) (layer "F.Cu") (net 7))
 (segment (start 138.488 63.2786) (end 139.7254 64.516) (width 0.25) (layer "F.Cu") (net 18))
 (segment (start 112.4204 93.6752) (end 114.1984 93.6752) (width 0.25) (layer "F.Cu") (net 18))
 (segment (start 139.7254 82.8548) (end 140.452 83.5814) (width 0.25) (layer "F.Cu") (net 18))
 (segment (start 114.1984 93.6752) (end 114.8842 92.9894) (width 0.25) (layer "F.Cu") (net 18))
 (segment (start 114.8842 64.590804) (end 116.196404 63.2786) (width 0.25) (layer "F.Cu") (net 18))
 (segment (start 140.452 83.5814) (end 142.4332 83.5814) (width 0.25) (layer "F.Cu") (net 18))
 (segment (start 114.8842 92.9894) (end 114.8842 64.590804) (width 0.25) (layer "F.Cu") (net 18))
 (segment (start 139.7254 64.516) (end 139.7254 82.8548) (width 0.25) (layer "F.Cu") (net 18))
 (segment (start 116.196404 63.2786) (end 138.488 63.2786) (width 0.25) (layer "F.Cu") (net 18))
 (segment (start 139.192 84.01157) (end 139.192 65.1002) (width 0.25) (layer "F.Cu") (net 20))
 (segment (start 137.8204 63.7286) (end 116.3828 63.7286) (width 0.25) (layer "F.Cu") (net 20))
 (segment (start 142.4332 86.1214) (end 141.30183 86.1214) (width 0.25) (layer "F.Cu") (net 20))
 (segment (start 115.3342 100.6928) (end 114.7318 101.2952) (width 0.25) (layer "F.Cu") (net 20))
 (segment (start 139.192 65.1002) (end 137.8204 63.7286) (width 0.25) (layer "F.Cu") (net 20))
 (segment (start 116.3828 63.7286) (end 115.3342 64.7772) (width 0.25) (layer "F.Cu") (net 20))
 (segment (start 115.3342 64.7772) (end 115.3342 100.6928) (width 0.25) (layer "F.Cu") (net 20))
 (segment (start 114.7318 101.2952) (end 112.4204 101.2952) (width 0.25) (layer "F.Cu") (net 20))
 (segment (start 141.30183 86.1214) (end 139.192 84.01157) (width 0.25) (layer "F.Cu") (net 20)))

